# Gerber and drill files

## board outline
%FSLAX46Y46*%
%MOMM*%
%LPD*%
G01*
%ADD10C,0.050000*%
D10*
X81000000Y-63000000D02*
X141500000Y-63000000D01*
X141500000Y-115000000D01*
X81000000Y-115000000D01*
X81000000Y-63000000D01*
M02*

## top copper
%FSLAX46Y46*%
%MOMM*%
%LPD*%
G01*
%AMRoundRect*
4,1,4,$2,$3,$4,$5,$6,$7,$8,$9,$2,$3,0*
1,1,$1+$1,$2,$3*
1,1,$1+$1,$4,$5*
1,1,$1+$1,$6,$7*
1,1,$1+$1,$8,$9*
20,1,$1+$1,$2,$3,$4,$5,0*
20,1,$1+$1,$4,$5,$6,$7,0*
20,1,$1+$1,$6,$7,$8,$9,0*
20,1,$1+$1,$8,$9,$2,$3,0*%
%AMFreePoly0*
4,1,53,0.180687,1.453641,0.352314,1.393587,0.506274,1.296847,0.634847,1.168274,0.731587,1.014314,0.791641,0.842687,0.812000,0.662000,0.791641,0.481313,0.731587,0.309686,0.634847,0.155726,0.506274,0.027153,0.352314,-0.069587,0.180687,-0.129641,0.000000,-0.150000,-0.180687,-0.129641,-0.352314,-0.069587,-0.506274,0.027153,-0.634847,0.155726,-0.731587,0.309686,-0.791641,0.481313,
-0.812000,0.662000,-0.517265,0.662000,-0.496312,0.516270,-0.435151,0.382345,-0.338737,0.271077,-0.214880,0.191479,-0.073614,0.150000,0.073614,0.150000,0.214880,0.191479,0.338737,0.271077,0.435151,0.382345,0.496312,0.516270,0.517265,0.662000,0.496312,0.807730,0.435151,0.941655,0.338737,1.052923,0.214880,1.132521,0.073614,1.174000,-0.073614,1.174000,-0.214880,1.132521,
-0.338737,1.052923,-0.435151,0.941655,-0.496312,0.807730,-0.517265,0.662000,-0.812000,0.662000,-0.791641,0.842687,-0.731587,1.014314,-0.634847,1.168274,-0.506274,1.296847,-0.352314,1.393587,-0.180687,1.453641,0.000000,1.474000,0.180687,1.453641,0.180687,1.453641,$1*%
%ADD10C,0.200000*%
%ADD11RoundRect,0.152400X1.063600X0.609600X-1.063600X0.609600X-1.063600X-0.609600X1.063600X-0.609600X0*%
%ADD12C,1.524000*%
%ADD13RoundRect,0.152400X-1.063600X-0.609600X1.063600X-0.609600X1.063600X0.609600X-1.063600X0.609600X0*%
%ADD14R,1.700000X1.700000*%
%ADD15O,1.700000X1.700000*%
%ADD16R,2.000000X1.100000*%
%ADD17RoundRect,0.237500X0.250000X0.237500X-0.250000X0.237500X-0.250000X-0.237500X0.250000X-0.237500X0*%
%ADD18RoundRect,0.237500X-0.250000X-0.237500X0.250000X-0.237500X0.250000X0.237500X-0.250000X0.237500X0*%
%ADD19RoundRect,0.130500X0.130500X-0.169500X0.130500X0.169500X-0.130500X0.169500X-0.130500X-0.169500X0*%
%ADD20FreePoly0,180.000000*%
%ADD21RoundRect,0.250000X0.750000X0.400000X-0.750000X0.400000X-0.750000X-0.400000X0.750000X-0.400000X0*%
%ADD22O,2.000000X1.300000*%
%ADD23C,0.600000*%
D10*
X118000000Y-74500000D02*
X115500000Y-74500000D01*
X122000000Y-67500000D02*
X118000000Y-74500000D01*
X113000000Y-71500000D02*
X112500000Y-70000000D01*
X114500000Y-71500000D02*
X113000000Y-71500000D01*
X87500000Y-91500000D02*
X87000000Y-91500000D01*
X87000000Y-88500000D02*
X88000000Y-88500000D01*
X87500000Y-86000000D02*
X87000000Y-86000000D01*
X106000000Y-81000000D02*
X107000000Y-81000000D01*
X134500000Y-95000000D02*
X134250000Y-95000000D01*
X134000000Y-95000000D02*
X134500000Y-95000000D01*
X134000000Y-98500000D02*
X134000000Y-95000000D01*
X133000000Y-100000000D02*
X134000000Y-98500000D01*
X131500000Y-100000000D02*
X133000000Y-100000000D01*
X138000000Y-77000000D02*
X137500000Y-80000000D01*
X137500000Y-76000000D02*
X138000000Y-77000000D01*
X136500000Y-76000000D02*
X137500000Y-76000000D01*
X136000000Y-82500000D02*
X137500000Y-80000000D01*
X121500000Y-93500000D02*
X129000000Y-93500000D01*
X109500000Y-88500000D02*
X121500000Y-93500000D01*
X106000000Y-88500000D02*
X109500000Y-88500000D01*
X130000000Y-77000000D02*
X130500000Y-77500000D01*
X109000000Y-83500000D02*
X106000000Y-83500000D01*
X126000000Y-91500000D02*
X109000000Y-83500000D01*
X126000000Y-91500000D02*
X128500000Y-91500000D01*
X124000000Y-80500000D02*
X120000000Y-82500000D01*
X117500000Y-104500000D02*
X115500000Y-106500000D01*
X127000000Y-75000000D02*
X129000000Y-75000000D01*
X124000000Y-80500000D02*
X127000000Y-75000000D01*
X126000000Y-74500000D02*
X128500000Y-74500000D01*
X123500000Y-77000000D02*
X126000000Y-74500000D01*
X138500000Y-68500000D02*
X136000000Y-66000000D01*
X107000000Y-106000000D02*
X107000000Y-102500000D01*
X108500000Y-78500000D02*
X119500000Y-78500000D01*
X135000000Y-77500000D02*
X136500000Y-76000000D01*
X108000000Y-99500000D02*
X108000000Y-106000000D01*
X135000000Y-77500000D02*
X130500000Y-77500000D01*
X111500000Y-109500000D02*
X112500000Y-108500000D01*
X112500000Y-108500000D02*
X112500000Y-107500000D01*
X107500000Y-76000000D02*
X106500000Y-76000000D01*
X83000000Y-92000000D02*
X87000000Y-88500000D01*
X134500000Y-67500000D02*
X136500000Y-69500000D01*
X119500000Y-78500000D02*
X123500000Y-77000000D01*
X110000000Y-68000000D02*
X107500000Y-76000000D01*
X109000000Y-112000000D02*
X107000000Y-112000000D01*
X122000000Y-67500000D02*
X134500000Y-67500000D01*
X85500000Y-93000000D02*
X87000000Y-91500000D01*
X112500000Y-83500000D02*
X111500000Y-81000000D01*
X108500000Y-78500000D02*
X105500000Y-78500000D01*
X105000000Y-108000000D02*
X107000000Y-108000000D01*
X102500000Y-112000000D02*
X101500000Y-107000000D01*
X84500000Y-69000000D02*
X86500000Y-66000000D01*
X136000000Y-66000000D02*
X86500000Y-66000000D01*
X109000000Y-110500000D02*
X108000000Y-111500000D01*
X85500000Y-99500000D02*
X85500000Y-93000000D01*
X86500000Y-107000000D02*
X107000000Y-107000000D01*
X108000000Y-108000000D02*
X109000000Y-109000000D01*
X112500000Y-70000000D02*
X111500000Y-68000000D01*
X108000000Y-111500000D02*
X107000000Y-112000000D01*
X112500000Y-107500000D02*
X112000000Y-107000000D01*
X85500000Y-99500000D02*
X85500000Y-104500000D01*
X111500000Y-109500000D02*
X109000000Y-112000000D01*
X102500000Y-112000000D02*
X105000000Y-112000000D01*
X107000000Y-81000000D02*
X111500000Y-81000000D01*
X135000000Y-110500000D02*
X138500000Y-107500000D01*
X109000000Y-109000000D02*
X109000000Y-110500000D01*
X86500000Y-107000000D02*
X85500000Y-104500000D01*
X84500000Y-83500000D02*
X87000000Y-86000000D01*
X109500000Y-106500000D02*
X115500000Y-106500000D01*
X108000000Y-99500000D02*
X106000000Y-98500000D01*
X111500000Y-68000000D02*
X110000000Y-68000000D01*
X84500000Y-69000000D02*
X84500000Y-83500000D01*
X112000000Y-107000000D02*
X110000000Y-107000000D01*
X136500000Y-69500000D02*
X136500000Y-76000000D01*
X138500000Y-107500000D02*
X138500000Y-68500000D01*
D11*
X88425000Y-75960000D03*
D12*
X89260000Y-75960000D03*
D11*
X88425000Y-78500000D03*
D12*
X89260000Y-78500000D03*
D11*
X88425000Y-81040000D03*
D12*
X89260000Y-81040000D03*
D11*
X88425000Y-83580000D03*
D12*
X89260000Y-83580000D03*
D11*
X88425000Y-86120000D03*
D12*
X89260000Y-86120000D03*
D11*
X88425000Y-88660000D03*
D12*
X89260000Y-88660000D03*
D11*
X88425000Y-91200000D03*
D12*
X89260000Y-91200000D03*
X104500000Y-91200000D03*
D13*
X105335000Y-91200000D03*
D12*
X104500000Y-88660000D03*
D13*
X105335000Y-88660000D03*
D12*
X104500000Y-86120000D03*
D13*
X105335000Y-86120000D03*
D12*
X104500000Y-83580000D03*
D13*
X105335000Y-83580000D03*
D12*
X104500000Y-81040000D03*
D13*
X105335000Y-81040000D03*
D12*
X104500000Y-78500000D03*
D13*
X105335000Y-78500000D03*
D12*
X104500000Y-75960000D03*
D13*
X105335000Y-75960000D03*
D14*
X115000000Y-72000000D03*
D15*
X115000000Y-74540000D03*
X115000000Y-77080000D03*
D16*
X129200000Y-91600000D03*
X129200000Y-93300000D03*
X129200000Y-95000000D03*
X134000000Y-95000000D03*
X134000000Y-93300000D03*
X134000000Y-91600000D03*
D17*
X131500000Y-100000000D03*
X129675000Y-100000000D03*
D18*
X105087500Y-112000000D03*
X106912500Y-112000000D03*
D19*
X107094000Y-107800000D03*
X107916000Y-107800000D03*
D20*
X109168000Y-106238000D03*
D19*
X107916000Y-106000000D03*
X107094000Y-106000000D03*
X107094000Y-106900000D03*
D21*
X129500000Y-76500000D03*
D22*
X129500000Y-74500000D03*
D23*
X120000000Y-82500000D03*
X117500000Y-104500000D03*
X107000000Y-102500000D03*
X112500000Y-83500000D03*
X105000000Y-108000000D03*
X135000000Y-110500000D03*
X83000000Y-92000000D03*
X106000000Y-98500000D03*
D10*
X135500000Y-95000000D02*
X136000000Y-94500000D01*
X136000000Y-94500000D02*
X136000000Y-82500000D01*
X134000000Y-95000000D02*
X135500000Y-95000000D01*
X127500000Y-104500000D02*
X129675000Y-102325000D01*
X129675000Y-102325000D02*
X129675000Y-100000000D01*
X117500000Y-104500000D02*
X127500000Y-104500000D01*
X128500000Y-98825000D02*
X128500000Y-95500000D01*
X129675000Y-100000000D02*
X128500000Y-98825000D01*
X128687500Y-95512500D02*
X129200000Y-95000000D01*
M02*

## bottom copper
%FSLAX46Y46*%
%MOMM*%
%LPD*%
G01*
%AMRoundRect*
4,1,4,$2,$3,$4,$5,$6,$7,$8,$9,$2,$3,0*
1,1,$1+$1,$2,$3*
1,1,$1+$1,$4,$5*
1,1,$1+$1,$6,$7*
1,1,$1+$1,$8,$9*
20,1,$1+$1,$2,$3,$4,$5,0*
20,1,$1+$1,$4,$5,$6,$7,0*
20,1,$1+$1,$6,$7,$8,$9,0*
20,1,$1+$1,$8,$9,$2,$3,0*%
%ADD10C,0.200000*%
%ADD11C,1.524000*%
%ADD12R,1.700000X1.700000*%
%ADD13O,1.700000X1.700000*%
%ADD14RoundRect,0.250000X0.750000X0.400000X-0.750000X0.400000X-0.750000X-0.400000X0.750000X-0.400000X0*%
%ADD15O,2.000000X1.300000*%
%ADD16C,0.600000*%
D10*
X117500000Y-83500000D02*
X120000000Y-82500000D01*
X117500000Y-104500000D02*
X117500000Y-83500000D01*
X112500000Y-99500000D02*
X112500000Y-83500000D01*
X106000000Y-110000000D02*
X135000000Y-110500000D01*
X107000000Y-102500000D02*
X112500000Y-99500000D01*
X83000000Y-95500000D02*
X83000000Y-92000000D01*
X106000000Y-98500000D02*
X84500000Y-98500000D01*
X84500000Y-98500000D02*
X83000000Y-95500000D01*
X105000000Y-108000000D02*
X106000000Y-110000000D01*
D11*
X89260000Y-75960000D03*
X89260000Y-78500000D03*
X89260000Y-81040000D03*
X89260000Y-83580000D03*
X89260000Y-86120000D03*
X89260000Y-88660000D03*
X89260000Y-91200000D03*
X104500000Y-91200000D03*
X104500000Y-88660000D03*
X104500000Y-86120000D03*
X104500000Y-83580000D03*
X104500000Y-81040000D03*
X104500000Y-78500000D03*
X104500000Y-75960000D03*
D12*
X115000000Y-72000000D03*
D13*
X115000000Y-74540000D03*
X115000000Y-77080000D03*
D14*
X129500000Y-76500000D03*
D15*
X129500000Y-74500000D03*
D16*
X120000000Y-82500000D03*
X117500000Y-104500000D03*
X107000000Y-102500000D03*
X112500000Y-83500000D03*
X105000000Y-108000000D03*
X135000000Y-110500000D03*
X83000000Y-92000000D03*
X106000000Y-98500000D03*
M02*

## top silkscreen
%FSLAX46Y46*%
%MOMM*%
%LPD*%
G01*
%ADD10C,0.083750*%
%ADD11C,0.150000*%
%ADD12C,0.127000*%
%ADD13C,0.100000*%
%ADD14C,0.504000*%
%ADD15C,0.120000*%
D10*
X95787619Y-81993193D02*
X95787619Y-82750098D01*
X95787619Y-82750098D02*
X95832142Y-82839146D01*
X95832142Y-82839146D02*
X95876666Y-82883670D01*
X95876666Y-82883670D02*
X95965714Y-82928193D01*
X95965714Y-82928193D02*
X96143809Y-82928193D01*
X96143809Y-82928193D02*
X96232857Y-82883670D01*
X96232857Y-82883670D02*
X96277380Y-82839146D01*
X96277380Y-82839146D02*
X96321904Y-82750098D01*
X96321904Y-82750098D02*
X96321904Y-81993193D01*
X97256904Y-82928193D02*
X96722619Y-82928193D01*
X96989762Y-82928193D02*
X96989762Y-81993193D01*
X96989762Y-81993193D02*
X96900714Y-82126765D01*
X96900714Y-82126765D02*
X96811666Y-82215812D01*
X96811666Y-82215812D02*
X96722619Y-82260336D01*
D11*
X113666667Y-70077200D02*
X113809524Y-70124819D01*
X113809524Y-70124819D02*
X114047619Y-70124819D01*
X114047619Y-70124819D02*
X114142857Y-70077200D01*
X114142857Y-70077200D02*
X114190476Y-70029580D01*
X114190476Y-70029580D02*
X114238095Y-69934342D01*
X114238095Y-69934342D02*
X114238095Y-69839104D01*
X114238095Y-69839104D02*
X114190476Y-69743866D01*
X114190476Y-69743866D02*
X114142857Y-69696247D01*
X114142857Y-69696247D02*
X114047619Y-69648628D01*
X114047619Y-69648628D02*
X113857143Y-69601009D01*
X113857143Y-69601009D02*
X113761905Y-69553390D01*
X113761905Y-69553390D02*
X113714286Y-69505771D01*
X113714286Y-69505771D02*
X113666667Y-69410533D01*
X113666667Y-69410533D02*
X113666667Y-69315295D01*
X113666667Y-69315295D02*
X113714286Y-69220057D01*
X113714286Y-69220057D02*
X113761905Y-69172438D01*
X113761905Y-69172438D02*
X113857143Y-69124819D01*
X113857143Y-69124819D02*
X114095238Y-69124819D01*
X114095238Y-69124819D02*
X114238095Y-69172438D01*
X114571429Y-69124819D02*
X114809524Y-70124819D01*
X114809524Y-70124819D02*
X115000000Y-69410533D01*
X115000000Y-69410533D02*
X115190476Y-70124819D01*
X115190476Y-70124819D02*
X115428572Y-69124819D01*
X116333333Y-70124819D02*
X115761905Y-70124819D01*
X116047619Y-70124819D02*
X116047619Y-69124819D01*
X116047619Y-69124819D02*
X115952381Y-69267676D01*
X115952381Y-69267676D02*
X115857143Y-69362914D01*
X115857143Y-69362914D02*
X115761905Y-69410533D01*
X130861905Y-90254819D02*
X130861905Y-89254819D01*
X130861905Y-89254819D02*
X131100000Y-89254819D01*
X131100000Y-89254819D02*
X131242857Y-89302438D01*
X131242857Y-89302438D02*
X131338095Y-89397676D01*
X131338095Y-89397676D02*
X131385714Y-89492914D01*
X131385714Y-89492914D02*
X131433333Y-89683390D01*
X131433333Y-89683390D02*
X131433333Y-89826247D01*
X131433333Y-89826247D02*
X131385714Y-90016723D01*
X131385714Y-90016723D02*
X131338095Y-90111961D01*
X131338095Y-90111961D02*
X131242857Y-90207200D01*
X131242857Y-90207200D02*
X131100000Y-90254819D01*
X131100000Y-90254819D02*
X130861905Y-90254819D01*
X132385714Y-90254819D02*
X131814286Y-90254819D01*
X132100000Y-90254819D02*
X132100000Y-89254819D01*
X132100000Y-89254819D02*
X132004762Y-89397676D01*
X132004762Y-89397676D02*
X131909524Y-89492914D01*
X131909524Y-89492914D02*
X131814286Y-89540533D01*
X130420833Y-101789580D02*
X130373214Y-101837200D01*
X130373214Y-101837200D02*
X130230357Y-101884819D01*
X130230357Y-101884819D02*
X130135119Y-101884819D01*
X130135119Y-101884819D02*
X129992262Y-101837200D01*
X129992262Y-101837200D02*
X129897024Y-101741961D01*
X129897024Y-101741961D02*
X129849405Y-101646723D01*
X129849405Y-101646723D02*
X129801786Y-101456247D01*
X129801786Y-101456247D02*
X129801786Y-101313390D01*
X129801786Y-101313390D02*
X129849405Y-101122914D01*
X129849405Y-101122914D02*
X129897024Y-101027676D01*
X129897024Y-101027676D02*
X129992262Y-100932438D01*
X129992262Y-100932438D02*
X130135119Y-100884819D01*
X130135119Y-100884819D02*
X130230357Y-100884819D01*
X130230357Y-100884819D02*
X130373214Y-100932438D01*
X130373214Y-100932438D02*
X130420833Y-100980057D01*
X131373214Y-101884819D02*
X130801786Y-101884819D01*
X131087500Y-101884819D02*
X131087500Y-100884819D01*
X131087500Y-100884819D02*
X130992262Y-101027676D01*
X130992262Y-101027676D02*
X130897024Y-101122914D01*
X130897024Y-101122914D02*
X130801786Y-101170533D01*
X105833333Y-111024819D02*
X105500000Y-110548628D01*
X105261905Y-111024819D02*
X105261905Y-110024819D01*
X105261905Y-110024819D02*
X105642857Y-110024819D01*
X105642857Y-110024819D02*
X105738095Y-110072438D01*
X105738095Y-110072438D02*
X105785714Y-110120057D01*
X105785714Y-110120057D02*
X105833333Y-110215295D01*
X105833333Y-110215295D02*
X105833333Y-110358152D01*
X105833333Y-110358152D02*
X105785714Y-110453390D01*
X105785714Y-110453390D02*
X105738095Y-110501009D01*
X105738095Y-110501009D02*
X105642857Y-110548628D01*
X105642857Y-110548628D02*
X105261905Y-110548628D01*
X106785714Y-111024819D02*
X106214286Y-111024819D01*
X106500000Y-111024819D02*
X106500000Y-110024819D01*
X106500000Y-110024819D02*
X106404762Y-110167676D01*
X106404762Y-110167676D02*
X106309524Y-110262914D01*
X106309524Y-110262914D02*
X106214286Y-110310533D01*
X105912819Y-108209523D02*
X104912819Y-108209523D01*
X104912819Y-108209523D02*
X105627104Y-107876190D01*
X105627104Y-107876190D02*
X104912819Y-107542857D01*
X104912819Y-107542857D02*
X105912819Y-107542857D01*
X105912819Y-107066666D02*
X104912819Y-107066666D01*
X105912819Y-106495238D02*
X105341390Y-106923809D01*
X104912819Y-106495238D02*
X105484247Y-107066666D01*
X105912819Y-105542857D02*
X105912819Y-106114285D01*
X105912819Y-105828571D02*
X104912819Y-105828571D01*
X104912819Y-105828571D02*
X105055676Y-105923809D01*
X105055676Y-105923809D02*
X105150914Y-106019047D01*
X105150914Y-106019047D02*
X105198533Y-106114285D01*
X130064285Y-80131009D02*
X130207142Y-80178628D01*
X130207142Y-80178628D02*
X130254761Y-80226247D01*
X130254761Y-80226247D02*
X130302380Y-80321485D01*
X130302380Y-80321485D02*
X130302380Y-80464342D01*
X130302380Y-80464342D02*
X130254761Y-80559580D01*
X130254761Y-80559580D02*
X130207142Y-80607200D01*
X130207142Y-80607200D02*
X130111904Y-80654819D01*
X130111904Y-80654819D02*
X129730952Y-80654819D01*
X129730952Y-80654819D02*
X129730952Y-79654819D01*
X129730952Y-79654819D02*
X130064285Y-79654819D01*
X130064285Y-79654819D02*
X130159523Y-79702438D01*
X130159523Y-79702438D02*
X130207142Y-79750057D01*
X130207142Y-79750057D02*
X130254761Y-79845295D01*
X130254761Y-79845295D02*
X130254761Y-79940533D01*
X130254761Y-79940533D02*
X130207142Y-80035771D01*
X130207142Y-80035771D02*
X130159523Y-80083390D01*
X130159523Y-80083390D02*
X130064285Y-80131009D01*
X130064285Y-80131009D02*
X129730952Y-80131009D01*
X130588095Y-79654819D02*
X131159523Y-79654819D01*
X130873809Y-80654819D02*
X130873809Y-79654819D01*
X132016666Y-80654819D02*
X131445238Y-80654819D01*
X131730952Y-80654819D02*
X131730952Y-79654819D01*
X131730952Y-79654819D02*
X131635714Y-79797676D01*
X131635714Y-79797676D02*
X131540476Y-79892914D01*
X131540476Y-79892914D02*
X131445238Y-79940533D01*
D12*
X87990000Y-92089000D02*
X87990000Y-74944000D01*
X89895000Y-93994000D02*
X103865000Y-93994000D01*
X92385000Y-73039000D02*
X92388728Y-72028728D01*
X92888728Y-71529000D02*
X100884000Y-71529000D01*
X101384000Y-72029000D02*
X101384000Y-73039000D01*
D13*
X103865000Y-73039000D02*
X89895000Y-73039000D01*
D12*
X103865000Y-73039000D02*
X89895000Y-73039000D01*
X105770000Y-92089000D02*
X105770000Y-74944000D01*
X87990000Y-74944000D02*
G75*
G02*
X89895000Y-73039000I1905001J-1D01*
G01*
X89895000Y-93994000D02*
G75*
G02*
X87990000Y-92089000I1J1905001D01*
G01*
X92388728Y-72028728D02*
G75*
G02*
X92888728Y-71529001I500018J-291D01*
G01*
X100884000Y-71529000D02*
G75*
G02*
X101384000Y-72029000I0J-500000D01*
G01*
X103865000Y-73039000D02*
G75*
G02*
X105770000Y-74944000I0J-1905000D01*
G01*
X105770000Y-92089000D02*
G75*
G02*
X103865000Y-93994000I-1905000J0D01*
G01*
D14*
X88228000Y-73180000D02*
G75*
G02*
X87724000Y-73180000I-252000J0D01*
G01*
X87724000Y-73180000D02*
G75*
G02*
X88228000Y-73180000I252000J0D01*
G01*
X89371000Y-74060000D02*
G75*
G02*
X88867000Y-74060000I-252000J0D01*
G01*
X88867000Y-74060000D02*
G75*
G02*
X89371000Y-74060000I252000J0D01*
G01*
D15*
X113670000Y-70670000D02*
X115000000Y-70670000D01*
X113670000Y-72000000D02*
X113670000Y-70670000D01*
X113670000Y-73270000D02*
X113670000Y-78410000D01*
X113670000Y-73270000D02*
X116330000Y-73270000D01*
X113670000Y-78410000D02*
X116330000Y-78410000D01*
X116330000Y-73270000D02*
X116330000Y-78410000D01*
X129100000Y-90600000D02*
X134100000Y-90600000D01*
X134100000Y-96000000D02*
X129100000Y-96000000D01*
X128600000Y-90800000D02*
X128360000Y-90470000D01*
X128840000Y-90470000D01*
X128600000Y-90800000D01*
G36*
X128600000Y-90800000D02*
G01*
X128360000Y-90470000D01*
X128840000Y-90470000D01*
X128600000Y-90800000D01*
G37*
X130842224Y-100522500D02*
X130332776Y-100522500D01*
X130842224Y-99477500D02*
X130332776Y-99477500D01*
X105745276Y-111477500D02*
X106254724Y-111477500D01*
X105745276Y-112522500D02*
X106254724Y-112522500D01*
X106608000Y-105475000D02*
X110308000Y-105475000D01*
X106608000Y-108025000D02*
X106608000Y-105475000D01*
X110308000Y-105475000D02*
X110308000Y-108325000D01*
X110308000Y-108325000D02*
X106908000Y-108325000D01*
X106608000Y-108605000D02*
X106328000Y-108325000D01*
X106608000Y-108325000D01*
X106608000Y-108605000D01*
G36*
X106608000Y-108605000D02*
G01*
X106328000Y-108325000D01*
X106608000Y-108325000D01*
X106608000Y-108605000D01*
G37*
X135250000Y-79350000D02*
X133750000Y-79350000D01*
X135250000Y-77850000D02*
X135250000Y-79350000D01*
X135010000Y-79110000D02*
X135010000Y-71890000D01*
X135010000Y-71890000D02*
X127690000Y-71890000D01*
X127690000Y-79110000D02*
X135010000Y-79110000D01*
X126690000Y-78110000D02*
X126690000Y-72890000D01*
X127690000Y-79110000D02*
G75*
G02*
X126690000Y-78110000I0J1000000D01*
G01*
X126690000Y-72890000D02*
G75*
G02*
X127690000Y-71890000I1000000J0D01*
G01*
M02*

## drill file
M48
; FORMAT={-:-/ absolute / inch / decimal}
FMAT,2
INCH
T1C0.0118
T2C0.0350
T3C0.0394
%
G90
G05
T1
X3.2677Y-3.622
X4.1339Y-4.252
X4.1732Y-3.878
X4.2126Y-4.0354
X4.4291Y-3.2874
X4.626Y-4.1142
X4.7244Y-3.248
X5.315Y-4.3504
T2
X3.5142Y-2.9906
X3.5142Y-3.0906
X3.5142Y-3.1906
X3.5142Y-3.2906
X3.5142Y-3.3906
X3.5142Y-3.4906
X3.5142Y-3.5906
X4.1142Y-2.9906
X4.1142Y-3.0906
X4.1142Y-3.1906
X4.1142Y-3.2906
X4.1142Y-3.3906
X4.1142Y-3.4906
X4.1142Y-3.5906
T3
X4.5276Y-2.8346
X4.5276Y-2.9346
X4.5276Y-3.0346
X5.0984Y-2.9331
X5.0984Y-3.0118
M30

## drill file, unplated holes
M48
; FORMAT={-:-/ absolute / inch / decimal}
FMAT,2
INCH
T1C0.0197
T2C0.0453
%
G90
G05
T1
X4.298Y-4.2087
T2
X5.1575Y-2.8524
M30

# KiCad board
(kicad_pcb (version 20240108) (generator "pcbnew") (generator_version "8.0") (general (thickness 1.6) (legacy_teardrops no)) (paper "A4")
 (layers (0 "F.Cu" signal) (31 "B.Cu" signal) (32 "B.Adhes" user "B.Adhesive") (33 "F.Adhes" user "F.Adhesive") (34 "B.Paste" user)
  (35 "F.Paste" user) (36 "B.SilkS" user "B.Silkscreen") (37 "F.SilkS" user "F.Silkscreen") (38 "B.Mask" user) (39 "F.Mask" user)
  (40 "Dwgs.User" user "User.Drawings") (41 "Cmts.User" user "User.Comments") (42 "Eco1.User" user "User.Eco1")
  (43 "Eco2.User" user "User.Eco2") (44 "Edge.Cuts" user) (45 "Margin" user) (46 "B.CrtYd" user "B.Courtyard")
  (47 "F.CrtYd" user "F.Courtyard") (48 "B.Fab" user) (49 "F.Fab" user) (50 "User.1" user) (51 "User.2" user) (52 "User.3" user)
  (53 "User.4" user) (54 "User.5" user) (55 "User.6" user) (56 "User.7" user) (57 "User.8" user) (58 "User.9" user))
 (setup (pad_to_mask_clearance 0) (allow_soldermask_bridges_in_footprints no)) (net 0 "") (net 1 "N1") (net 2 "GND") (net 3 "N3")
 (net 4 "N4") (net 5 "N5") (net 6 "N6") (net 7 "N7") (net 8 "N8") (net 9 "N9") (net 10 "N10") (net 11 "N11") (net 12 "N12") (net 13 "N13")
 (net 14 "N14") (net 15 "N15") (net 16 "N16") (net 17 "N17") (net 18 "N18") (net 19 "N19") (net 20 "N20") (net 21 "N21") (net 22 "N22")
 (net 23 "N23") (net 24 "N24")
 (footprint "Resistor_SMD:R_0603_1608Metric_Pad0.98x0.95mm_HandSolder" (layer "F.Cu") (at 130.5875 100 180)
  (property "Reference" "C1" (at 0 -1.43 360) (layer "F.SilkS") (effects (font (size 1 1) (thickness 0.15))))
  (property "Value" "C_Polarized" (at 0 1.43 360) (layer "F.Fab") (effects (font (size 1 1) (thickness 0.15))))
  (fp_line (start -0.254724 0.5225) (end 0.254724 0.5225) (stroke (width 0.12) (type solid)) (layer "F.SilkS"))
  (fp_line (start -0.254724 -0.5225) (end 0.254724 -0.5225) (stroke (width 0.12) (type solid)) (layer "F.SilkS"))
  (pad "1" smd roundrect (at -0.9125 0 180) (size 0.975 0.95) (layers "F.Cu" "F.Paste" "F.Mask") (roundrect_rratio 0.25) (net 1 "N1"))
  (pad "2" smd roundrect (at 0.9125 0 180) (size 0.975 0.95) (layers "F.Cu" "F.Paste" "F.Mask") (roundrect_rratio 0.25) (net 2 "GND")))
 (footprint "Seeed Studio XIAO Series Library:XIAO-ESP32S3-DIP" (layer "F.Cu") (at 96.88 83.58)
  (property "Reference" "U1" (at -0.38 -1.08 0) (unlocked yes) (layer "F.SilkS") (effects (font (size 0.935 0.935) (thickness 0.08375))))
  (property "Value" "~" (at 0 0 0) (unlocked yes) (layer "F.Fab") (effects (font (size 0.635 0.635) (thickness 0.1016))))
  (fp_line (start -8.89 8.509) (end -8.89 -8.636) (stroke (width 0.127) (type solid)) (layer "F.SilkS"))
  (fp_line (start -6.985 10.414) (end 6.985 10.414) (stroke (width 0.127) (type solid)) (layer "F.SilkS"))
  (fp_line (start -4.495 -10.541) (end -4.491272 -11.551272) (stroke (width 0.127) (type solid)) (layer "F.SilkS"))
  (fp_line (start -3.991272 -12.051) (end 4.004 -12.051) (stroke (width 0.127) (type solid)) (layer "F.SilkS"))
  (fp_line (start 4.504 -11.551) (end 4.504 -10.541) (stroke (width 0.127) (type solid)) (layer "F.SilkS"))
  (fp_line (start 6.985 -10.541) (end -6.985 -10.541) (stroke (width 0.1) (type solid)) (layer "F.SilkS"))
  (fp_line (start 6.985 -10.541) (end -6.985 -10.541) (stroke (width 0.127) (type solid)) (layer "F.SilkS"))
  (fp_line (start 8.89 8.509) (end 8.89 -8.636) (stroke (width 0.127) (type solid)) (layer "F.SilkS"))
  (fp_arc (start -8.89 -8.636) (mid -8.332038 -9.983038) (end -6.985 -10.541) (stroke (width 0.127) (type solid)) (layer "F.SilkS"))
  (fp_arc (start -6.985 10.414) (mid -8.332038 9.856038) (end -8.89 8.509) (stroke (width 0.127) (type solid)) (layer "F.SilkS"))
  (fp_arc (start -4.491272 -11.551272) (mid -4.344724 -11.904644) (end -3.991272 -12.051) (stroke (width 0.127) (type default))
   (layer "F.SilkS"))
  (fp_arc (start 4.004 -12.051) (mid 4.357553 -11.904553) (end 4.504 -11.551) (stroke (width 0.127) (type default)) (layer "F.SilkS"))
  (fp_arc (start 6.985 -10.541) (mid 8.332038 -9.983038) (end 8.89 -8.636) (stroke (width 0.127) (type solid)) (layer "F.SilkS"))
  (fp_arc (start 8.89 8.509) (mid 8.332038 9.856038) (end 6.985 10.414) (stroke (width 0.127) (type solid)) (layer "F.SilkS"))
  (fp_circle (center -8.904 -10.4) (end -8.904 -10.654) (stroke (width 0.5) (type solid)) (fill solid) (layer "F.SilkS"))
  (fp_circle (center -7.761 -9.52) (end -7.761 -9.774) (stroke (width 0.5) (type solid)) (fill solid) (layer "F.SilkS"))
  (pad "1" smd roundrect (at -8.455 -7.62 180) (size 2.432 1.524) (layers "F.Cu" "F.Mask") (roundrect_rratio 0.1) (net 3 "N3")
   (thermal_bridge_angle 45))
  (pad "1" thru_hole circle (at -7.62 -7.62 180) (size 1.524 1.524) (drill 0.889) (layers "*.Cu" "*.Mask") (remove_unused_layers no)
   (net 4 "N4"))
  (pad "2" smd roundrect (at -8.455 -5.08 180) (size 2.432 1.524) (layers "F.Cu" "F.Mask") (roundrect_rratio 0.1) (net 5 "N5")
   (thermal_bridge_angle 45))
  (pad "2" thru_hole circle (at -7.62 -5.08 180) (size 1.524 1.524) (drill 0.889) (layers "*.Cu" "*.Mask") (remove_unused_layers no)
   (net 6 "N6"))
  (pad "3" smd roundrect (at -8.455 -2.54 180) (size 2.432 1.524) (layers "F.Cu" "F.Mask") (roundrect_rratio 0.1) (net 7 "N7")
   (thermal_bridge_angle 45))
  (pad "3" thru_hole circle (at -7.62 -2.54 180) (size 1.524 1.524) (drill 0.889) (layers "*.Cu" "*.Mask") (remove_unused_layers no)
   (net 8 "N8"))
  (pad "4" smd roundrect (at -8.455 0 180) (size 2.432 1.524) (layers "F.Cu" "F.Mask") (roundrect_rratio 0.1) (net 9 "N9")
   (thermal_bridge_angle 45))
  (pad "4" thru_hole circle (at -7.62 0 180) (size 1.524 1.524) (drill 0.889) (layers "*.Cu" "*.Mask") (remove_unused_layers no)
   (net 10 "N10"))
  (pad "5" smd roundrect (at -8.455 2.54 180) (size 2.432 1.524) (layers "F.Cu" "F.Mask") (roundrect_rratio 0.1) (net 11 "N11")
   (thermal_bridge_angle 45))
  (pad "5" thru_hole circle (at -7.62 2.54 180) (size 1.524 1.524) (drill 0.889) (layers "*.Cu" "*.Mask") (remove_unused_layers no)
   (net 11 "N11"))
  (pad "6" smd roundrect (at -8.455 5.08 180) (size 2.432 1.524) (layers "F.Cu" "F.Mask") (roundrect_rratio 0.1) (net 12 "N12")
   (thermal_bridge_angle 45))
  (pad "6" thru_hole circle (at -7.62 5.08 180) (size 1.524 1.524) (drill 0.889) (layers "*.Cu" "*.Mask") (remove_unused_layers no)
   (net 12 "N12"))
  (pad "7" smd roundrect (at -8.455 7.62 180) (size 2.432 1.524) (layers "F.Cu" "F.Mask") (roundrect_rratio 0.1) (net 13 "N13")
   (thermal_bridge_angle 45))
  (pad "7" thru_hole circle (at -7.62 7.62 180) (size 1.524 1.524) (drill 0.889) (layers "*.Cu" "*.Mask") (remove_unused_layers no)
   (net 13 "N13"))
  (pad "8" thru_hole circle (at 7.62 7.62) (size 1.524 1.524) (drill 0.889) (layers "*.Cu" "*.Mask") (remove_unused_layers no)
   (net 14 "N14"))
  (pad "8" smd roundrect (at 8.455 7.62) (size 2.432 1.524) (layers "F.Cu" "F.Mask") (roundrect_rratio 0.1) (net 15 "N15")
   (thermal_bridge_angle 45))
  (pad "9" thru_hole circle (at 7.62 5.08) (size 1.524 1.524) (drill 0.889) (layers "*.Cu" "*.Mask") (remove_unused_layers no)
   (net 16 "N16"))
  (pad "9" smd roundrect (at 8.455 5.08) (size 2.432 1.524) (layers "F.Cu" "F.Mask") (roundrect_rratio 0.1) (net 16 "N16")
   (thermal_bridge_angle 45))
  (pad "10" thru_hole circle (at 7.62 2.54) (size 1.524 1.524) (drill 0.889) (layers "*.Cu" "*.Mask") (remove_unused_layers no)
   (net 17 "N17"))
  (pad "10" smd roundrect (at 8.455 2.54) (size 2.432 1.524) (layers "F.Cu" "F.Mask") (roundrect_rratio 0.1) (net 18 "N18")
   (thermal_bridge_angle 45))
  (pad "11" thru_hole circle (at 7.62 0) (size 1.524 1.524) (drill 0.889) (layers "*.Cu" "*.Mask") (remove_unused_layers no) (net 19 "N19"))
  (pad "11" smd roundrect (at 8.455 0) (size 2.432 1.524) (layers "F.Cu" "F.Mask") (roundrect_rratio 0.1) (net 19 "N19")
   (thermal_bridge_angle 45))
  (pad "12" thru_hole circle (at 7.62 -2.54) (size 1.524 1.524) (drill 0.889) (layers "*.Cu" "*.Mask") (remove_unused_layers no)
   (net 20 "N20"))
  (pad "12" smd roundrect (at 8.455 -2.54) (size 2.432 1.524) (layers "F.Cu" "F.Mask") (roundrect_rratio 0.1) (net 20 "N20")
   (thermal_bridge_angle 45))
  (pad "13" thru_hole circle (at 7.62 -5.08) (size 1.524 1.524) (drill 0.889) (layers "*.Cu" "*.Mask") (remove_unused_layers no)
   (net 2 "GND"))
  (pad "13" smd roundrect (at 8.455 -5.08) (size 2.432 1.524) (layers "F.Cu" "F.Mask") (roundrect_rratio 0.1) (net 2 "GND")
   (thermal_bridge_angle 45))
  (pad "14" thru_hole circle (at 7.62 -7.62) (size 1.524 1.524) (drill 0.889) (layers "*.Cu" "*.Mask") (remove_unused_layers no)
   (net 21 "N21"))
  (pad "14" smd roundrect (at 8.455 -7.62) (size 2.432 1.524) (layers "F.Cu" "F.Mask") (roundrect_rratio 0.1) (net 21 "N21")
   (thermal_bridge_angle 45)))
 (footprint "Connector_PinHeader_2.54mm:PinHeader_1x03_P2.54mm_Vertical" (layer "F.Cu") (at 115 72)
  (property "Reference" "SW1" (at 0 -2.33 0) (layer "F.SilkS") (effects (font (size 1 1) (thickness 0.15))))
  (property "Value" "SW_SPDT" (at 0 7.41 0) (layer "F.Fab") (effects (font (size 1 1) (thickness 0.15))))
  (fp_line (start -1.33 -1.33) (end 0 -1.33) (stroke (width 0.12) (type solid)) (layer "F.SilkS"))
  (fp_line (start -1.33 0) (end -1.33 -1.33) (stroke (width 0.12) (type solid)) (layer "F.SilkS"))
  (fp_line (start -1.33 1.27) (end -1.33 6.41) (stroke (width 0.12) (type solid)) (layer "F.SilkS"))
  (fp_line (start -1.33 1.27) (end 1.33 1.27) (stroke (width 0.12) (type solid)) (layer "F.SilkS"))
  (fp_line (start -1.33 6.41) (end 1.33 6.41) (stroke (width 0.12) (type solid)) (layer "F.SilkS"))
  (fp_line (start 1.33 1.27) (end 1.33 6.41) (stroke (width 0.12) (type solid)) (layer "F.SilkS"))
  (pad "1" thru_hole rect (at 0 0) (size 1.7 1.7) (drill 1) (layers "*.Cu" "*.Mask") (remove_unused_layers no) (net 21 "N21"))
  (pad "2" thru_hole oval (at 0 2.54) (size 1.7 1.7) (drill 1) (layers "*.Cu" "*.Mask") (remove_unused_layers no) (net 1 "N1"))
  (pad "3" thru_hole oval (at 0 5.08) (size 1.7 1.7) (drill 1) (layers "*.Cu" "*.Mask") (remove_unused_layers no) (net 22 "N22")))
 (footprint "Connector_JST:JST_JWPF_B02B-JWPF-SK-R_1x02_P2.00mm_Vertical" (layer "F.Cu") (at 129.5 76.5 180)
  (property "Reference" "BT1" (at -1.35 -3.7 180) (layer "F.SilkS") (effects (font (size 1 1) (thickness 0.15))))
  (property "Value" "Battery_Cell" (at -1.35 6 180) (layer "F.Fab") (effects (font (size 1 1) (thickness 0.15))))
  (fp_line (start 2.81 -1.61) (end 2.81 3.61) (stroke (width 0.12) (type solid)) (layer "F.SilkS"))
  (fp_line (start 1.81 -2.61) (end -5.51 -2.61) (stroke (width 0.12) (type solid)) (layer "F.SilkS"))
  (fp_line (start -5.51 4.61) (end 1.81 4.61) (stroke (width 0.12) (type solid)) (layer "F.SilkS"))
  (fp_line (start -5.51 -2.61) (end -5.51 4.61) (stroke (width 0.12) (type solid)) (layer "F.SilkS"))
  (fp_line (start -5.75 -1.35) (end -5.75 -2.85) (stroke (width 0.12) (type solid)) (layer "F.SilkS"))
  (fp_line (start -5.75 -2.85) (end -4.25 -2.85) (stroke (width 0.12) (type solid)) (layer "F.SilkS"))
  (fp_arc (start 2.81 3.61) (mid 2.517107 4.317107) (end 1.81 4.61) (stroke (width 0.12) (type solid)) (layer "F.SilkS"))
  (fp_arc (start 1.81 -2.61) (mid 2.517107 -2.317107) (end 2.81 -1.61) (stroke (width 0.12) (type solid)) (layer "F.SilkS"))
  (pad "" np_thru_hole circle (at -1.5 4.05 180) (size 1.15 1.15) (drill 1.15) (layers "*.Cu" "*.Mask"))
  (pad "1" thru_hole roundrect (at 0 0 180) (size 2 1.3) (drill 1) (layers "*.Cu" "*.Mask") (remove_unused_layers no)
   (roundrect_rratio 0.192308) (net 1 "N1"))
  (pad "2" thru_hole oval (at 0 2 180) (size 2 1.3) (drill 1) (layers "*.Cu" "*.Mask") (remove_unused_layers no) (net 2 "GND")))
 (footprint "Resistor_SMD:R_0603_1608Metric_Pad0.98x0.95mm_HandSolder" (layer "F.Cu") (at 106 112)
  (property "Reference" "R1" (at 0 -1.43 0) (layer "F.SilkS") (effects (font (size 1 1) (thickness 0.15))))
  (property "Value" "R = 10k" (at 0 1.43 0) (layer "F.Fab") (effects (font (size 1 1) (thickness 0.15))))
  (fp_line (start -0.254724 -0.5225) (end 0.254724 -0.5225) (stroke (width 0.12) (type solid)) (layer "F.SilkS"))
  (fp_line (start -0.254724 0.5225) (end 0.254724 0.5225) (stroke (width 0.12) (type solid)) (layer "F.SilkS"))
  (pad "1" smd roundrect (at -0.9125 0) (size 0.975 0.95) (layers "F.Cu" "F.Paste" "F.Mask") (roundrect_rratio 0.25) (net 13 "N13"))
  (pad "2" smd roundrect (at 0.9125 0) (size 0.975 0.95) (layers "F.Cu" "F.Paste" "F.Mask") (roundrect_rratio 0.25) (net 2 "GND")))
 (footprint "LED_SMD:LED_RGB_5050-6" (layer "F.Cu") (at 131.6 93.3)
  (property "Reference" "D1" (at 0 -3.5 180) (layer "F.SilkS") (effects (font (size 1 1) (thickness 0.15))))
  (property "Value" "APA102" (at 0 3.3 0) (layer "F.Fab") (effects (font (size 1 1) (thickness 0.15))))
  (fp_line (start -2.5 -2.7) (end 2.5 -2.7) (stroke (width 0.12) (type solid)) (layer "F.SilkS"))
  (fp_line (start 2.5 2.7) (end -2.5 2.7) (stroke (width 0.12) (type solid)) (layer "F.SilkS"))
  (fp_poly
   (pts (xy -3 -2.5) (xy -3.24 -2.83) (xy -2.76 -2.83) (xy -3 -2.5)) (stroke (width 0.12) (type solid)) (fill solid) (layer "F.SilkS"))
  (pad "1" smd rect (at -2.4 -1.7 90) (size 1.1 2) (layers "F.Cu" "F.Paste" "F.Mask") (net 19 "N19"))
  (pad "2" smd rect (at -2.4 0 90) (size 1.1 2) (layers "F.Cu" "F.Paste" "F.Mask") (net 16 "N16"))
  (pad "3" smd rect (at -2.4 1.7 90) (size 1.1 2) (layers "F.Cu" "F.Paste" "F.Mask") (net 2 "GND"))
  (pad "4" smd rect (at 2.4 1.7 90) (size 1.1 2) (layers "F.Cu" "F.Paste" "F.Mask") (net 1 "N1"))
  (pad "5" smd rect (at 2.4 0 90) (size 1.1 2) (layers "F.Cu" "F.Paste" "F.Mask") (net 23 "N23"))
  (pad "6" smd rect (at 2.4 -1.7 90) (size 1.1 2) (layers "F.Cu" "F.Paste" "F.Mask") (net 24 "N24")))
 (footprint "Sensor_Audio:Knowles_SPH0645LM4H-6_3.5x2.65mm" (layer "F.Cu") (at 108.458 106.9 90)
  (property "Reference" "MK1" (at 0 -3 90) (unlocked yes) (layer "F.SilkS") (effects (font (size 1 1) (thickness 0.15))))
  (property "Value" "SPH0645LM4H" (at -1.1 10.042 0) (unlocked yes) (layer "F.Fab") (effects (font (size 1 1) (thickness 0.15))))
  (fp_line (start 1.425 -1.85) (end 1.425 1.85) (stroke (width 0.12) (type default)) (layer "F.SilkS"))
  (fp_line (start -1.125 -1.85) (end 1.425 -1.85) (stroke (width 0.12) (type default)) (layer "F.SilkS"))
  (fp_line (start 1.425 1.85) (end -1.425 1.85) (stroke (width 0.12) (type default)) (layer "F.SilkS"))
  (fp_line (start -1.425 1.85) (end -1.425 -1.55) (stroke (width 0.12) (type default)) (layer "F.SilkS"))
  (fp_poly
   (pts (xy -1.425 -1.85) (xy -1.705 -1.85) (xy -1.425 -2.13) (xy -1.425 -1.85)) (stroke (width 0.12) (type solid)) (fill solid)
   (layer "F.SilkS"))
  (pad "" np_thru_hole circle (at 0 0.71 90) (size 0.5 0.5) (drill 0.5) (layers "*.Mask"))
  (pad "1" smd roundrect (at -0.9 -1.364 90) (size 0.6 0.522) (layers "F.Cu" "F.Paste" "F.Mask") (roundrect_rratio 0.25) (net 11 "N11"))
  (pad "2" smd roundrect (at -0.9 -0.542 90) (size 0.6 0.522) (layers "F.Cu" "F.Paste" "F.Mask") (roundrect_rratio 0.25) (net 2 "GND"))
  (pad "3" smd custom (at 0.662 0.71 180) (size 0.3 0.3) (layers "F.Cu" "F.Mask") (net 2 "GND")
   (options (clearance outline) (anchor circle)) (primitives))
  (pad "4" smd roundrect (at 0.9 -0.542 90) (size 0.6 0.522) (layers "F.Cu" "F.Paste" "F.Mask") (roundrect_rratio 0.25) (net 12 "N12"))
  (pad "5" smd roundrect (at 0.9 -1.364 90) (size 0.6 0.522) (layers "F.Cu" "F.Paste" "F.Mask") (roundrect_rratio 0.25) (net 20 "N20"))
  (pad "6" smd roundrect (at 0 -1.364 90) (size 0.6 0.522) (layers "F.Cu" "F.Paste" "F.Mask") (roundrect_rratio 0.25) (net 13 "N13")))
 (gr_line (start 137.5 76) (end 138 77) (stroke (width 0.2) (type default)) (layer "F.Cu") (net 1))
 (gr_line (start 106 88.5) (end 109.5 88.5) (stroke (width 0.2) (type default)) (layer "F.Cu") (net 16))
 (gr_line (start 138.5 68.5) (end 136 66) (stroke (width 0.2) (type default)) (layer "F.Cu") (net 11))
 (gr_line (start 126 91.5) (end 109 83.5) (stroke (width 0.2) (type default)) (layer "F.Cu") (net 19))
 (gr_line (start 124 80.5) (end 127 75) (stroke (width 0.2) (type default)) (layer "F.Cu") (net 2))
 (gr_line (start 107 106) (end 107 102.5) (stroke (width 0.2) (type default)) (layer "F.Cu") (net 20))
 (gr_line (start 134 95) (end 134.5 95) (stroke (width 0.2) (type default)) (layer "F.Cu") (net 1))
 (gr_line (start 108.5 78.5) (end 119.5 78.5) (stroke (width 0.2) (type default)) (layer "F.Cu") (net 2))
 (gr_line (start 135 77.5) (end 136.5 76) (stroke (width 0.2) (type default)) (layer "F.Cu") (net 1))
 (gr_line (start 108 99.5) (end 108 106) (stroke (width 0.2) (type default)) (layer "F.Cu") (net 12))
 (gr_line (start 135 77.5) (end 130.5 77.5) (stroke (width 0.2) (type default)) (layer "F.Cu") (net 1))
 (gr_line (start 109.5 88.5) (end 121.5 93.5) (stroke (width 0.2) (type default)) (layer "F.Cu") (net 16))
 (gr_line (start 111.5 109.5) (end 112.5 108.5) (stroke (width 0.2) (type default)) (layer "F.Cu") (net 2))
 (gr_line (start 112.5 108.5) (end 112.5 107.5) (stroke (width 0.2) (type default)) (layer "F.Cu") (net 2))
 (gr_line (start 127 75) (end 129 75) (stroke (width 0.2) (type default)) (layer "F.Cu") (net 2))
 (gr_line (start 123.5 77) (end 126 74.5) (stroke (width 0.2) (type default)) (layer "F.Cu") (net 2))
 (gr_line (start 107.5 76) (end 106.5 76) (stroke (width 0.2) (type default)) (layer "F.Cu") (net 21))
 (gr_line (start 83 92) (end 87 88.5) (stroke (width 0.2) (type default)) (layer "F.Cu") (net 12))
 (gr_line (start 134.5 67.5) (end 136.5 69.5) (stroke (width 0.2) (type default)) (layer "F.Cu") (net 1))
 (gr_line (start 119.5 78.5) (end 123.5 77) (stroke (width 0.2) (type default)) (layer "F.Cu") (net 2))
 (gr_line (start 110 68) (end 107.5 76) (stroke (width 0.2) (type default)) (layer "F.Cu") (net 21))
 (gr_line (start 121.5 93.5) (end 129 93.5) (stroke (width 0.2) (type default)) (layer "F.Cu") (net 16))
 (gr_line (start 109 83.5) (end 106 83.5) (stroke (width 0.2) (type default)) (layer "F.Cu") (net 19))
 (gr_line (start 109 112) (end 107 112) (stroke (width 0.2) (type default)) (layer "F.Cu") (net 2))
 (gr_line (start 106 81) (end 107 81) (stroke (width 0.2) (type default)) (layer "F.Cu") (net 20))
 (gr_line (start 117.5 104.5) (end 115.5 106.5) (stroke (width 0.2) (type default)) (layer "F.Cu") (net 2))
 (gr_line (start 122 67.5) (end 134.5 67.5) (stroke (width 0.2) (type default)) (layer "F.Cu") (net 1))
 (gr_line (start 85.5 93) (end 87 91.5) (stroke (width 0.2) (type default)) (layer "F.Cu") (net 13))
 (gr_line (start 136 82.5) (end 137.5 80) (stroke (width 0.2) (type default)) (layer "F.Cu") (net 1))
 (gr_line (start 112.5 83.5) (end 111.5 81) (stroke (width 0.2) (type default)) (layer "F.Cu") (net 20))
 (gr_line (start 108.5 78.5) (end 105.5 78.5) (stroke (width 0.2) (type default)) (layer "F.Cu") (net 2))
 (gr_line (start 105 108) (end 107 108) (stroke (width 0.2) (type default)) (layer "F.Cu") (net 11))
 (gr_line (start 138 77) (end 137.5 80) (stroke (width 0.2) (type default)) (layer "F.Cu") (net 1))
 (gr_line (start 102.5 112) (end 101.5 107) (stroke (width 0.2) (type default)) (layer "F.Cu") (net 13))
 (gr_line (start 134.5 95) (end 134.25 95) (stroke (width 0.2) (type default)) (layer "F.Cu") (net 1))
 (gr_line (start 84.5 69) (end 86.5 66) (stroke (width 0.2) (type default)) (layer "F.Cu") (net 11))
 (gr_line (start 136 66) (end 86.5 66) (stroke (width 0.2) (type default)) (layer "F.Cu") (net 11))
 (gr_line (start 87.5 86) (end 87 86) (stroke (width 0.2) (type default)) (layer "F.Cu") (net 11))
 (gr_line (start 131.5 100) (end 133 100) (stroke (width 0.2) (type default)) (layer "F.Cu") (net 1))
 (gr_line (start 126 91.5) (end 128.5 91.5) (stroke (width 0.2) (type default)) (layer "F.Cu") (net 19))
 (gr_line (start 109 110.5) (end 108 111.5) (stroke (width 0.2) (type default)) (layer "F.Cu") (net 2))
 (gr_line (start 85.5 99.5) (end 85.5 93) (stroke (width 0.2) (type default)) (layer "F.Cu") (net 13))
 (gr_line (start 86.5 107) (end 107 107) (stroke (width 0.2) (type default)) (layer "F.Cu") (net 13))
 (gr_line (start 134 98.5) (end 134 95) (stroke (width 0.2) (type default)) (layer "F.Cu") (net 1))
 (gr_line (start 108 108) (end 109 109) (stroke (width 0.2) (type default)) (layer "F.Cu") (net 2))
 (gr_line (start 112.5 70) (end 111.5 68) (stroke (width 0.2) (type default)) (layer "F.Cu") (net 21))
 (gr_line (start 136.5 76) (end 137.5 76) (stroke (width 0.2) (type default)) (layer "F.Cu") (net 1))
 (gr_line (start 87 88.5) (end 88 88.5) (stroke (width 0.2) (type default)) (layer "F.Cu") (net 12))
 (gr_line (start 108 111.5) (end 107 112) (stroke (width 0.2) (type default)) (layer "F.Cu") (net 2))
 (gr_line (start 112.5 107.5) (end 112 107) (stroke (width 0.2) (type default)) (layer "F.Cu") (net 2))
 (gr_line (start 85.5 99.5) (end 85.5 104.5) (stroke (width 0.2) (type default)) (layer "F.Cu") (net 13))
 (gr_line (start 111.5 109.5) (end 109 112) (stroke (width 0.2) (type default)) (layer "F.Cu") (net 2))
 (gr_line (start 133 100) (end 134 98.5) (stroke (width 0.2) (type default)) (layer "F.Cu") (net 1))
 (gr_line (start 114.5 71.5) (end 113 71.5) (stroke (width 0.2) (type default)) (layer "F.Cu") (net 21))
 (gr_line (start 102.5 112) (end 105 112) (stroke (width 0.2) (type default)) (layer "F.Cu") (net 13))
 (gr_line (start 107 81) (end 111.5 81) (stroke (width 0.2) (type default)) (layer "F.Cu") (net 20))
 (gr_line (start 126 74.5) (end 128.5 74.5) (stroke (width 0.2) (type default)) (layer "F.Cu") (net 2))
 (gr_line (start 135 110.5) (end 138.5 107.5) (stroke (width 0.2) (type default)) (layer "F.Cu") (net 11))
 (gr_line (start 109 109) (end 109 110.5) (stroke (width 0.2) (type default)) (layer "F.Cu") (net 2))
 (gr_line (start 86.5 107) (end 85.5 104.5) (stroke (width 0.2) (type default)) (layer "F.Cu") (net 13))
 (gr_line (start 118 74.5) (end 115.5 74.5) (stroke (width 0.2) (type default)) (layer "F.Cu") (net 1))
 (gr_line (start 87.5 91.5) (end 87 91.5) (stroke (width 0.2) (type default)) (layer "F.Cu") (net 13))
 (gr_line (start 122 67.5) (end 118 74.5) (stroke (width 0.2) (type default)) (layer "F.Cu") (net 1))
 (gr_line (start 84.5 83.5) (end 87 86) (stroke (width 0.2) (type default)) (layer "F.Cu") (net 11))
 (gr_line (start 109.5 106.5) (end 115.5 106.5) (stroke (width 0.2) (type default)) (layer "F.Cu") (net 2))
 (gr_line (start 108 99.5) (end 106 98.5) (stroke (width 0.2) (type default)) (layer "F.Cu") (net 12))
 (gr_line (start 113 71.5) (end 112.5 70) (stroke (width 0.2) (type default)) (layer "F.Cu") (net 21))
 (gr_line (start 111.5 68) (end 110 68) (stroke (width 0.2) (type default)) (layer "F.Cu") (net 21))
 (gr_line (start 130 77) (end 130.5 77.5) (stroke (width 0.2) (type default)) (layer "F.Cu") (net 1))
 (gr_line (start 84.5 69) (end 84.5 83.5) (stroke (width 0.2) (type default)) (layer "F.Cu") (net 11))
 (gr_line (start 124 80.5) (end 120 82.5) (stroke (width 0.2) (type default)) (layer "F.Cu") (net 2))
 (gr_line (start 112 107) (end 110 107) (stroke (width 0.2) (type default)) (layer "F.Cu") (net 2))
 (gr_line (start 136.5 69.5) (end 136.5 76) (stroke (width 0.2) (type default)) (layer "F.Cu") (net 1))
 (gr_line (start 138.5 107.5) (end 138.5 68.5) (stroke (width 0.2) (type default)) (layer "F.Cu") (net 11))
 (gr_line (start 117.5 83.5) (end 120 82.5) (stroke (width 0.2) (type default)) (layer "B.Cu") (net 2))
 (gr_line (start 112.5 99.5) (end 112.5 83.5) (stroke (width 0.2) (type default)) (layer "B.Cu") (net 20))
 (gr_line (start 106 110) (end 135 110.5) (stroke (width 0.2) (type default)) (layer "B.Cu") (net 11))
 (gr_line (start 107 102.5) (end 112.5 99.5) (stroke (width 0.2) (type default)) (layer "B.Cu") (net 20))
 (gr_line (start 83 95.5) (end 83 92) (stroke (width 0.2) (type default)) (layer "B.Cu") (net 12))
 (gr_line (start 106 98.5) (end 84.5 98.5) (stroke (width 0.2) (type default)) (layer "B.Cu") (net 12))
 (gr_line (start 84.5 98.5) (end 83 95.5) (stroke (width 0.2) (type default)) (layer "B.Cu") (net 12))
 (gr_line (start 105 108) (end 106 110) (stroke (width 0.2) (type default)) (layer "B.Cu") (net 11))
 (gr_line (start 117.5 104.5) (end 117.5 83.5) (stroke (width 0.2) (type default)) (layer "B.Cu") (net 2))
 (gr_rect (start 81 63) (end 141.5 115) (stroke (width 0.05) (type default)) (fill none) (layer "Edge.Cuts"))
 (via (at 107 102.5) (size 0.6) (drill 0.3) (layers "F.Cu" "B.Cu") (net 20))
 (via (at 112.5 83.5) (size 0.6) (drill 0.3) (layers "F.Cu" "B.Cu") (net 20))
 (via (at 105 108) (size 0.6) (drill 0.3) (layers "F.Cu" "B.Cu") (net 11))
 (via (at 135 110.5) (size 0.6) (drill 0.3) (layers "F.Cu" "B.Cu") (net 11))
 (via (at 83 92) (size 0.6) (drill 0.3) (layers "F.Cu" "B.Cu") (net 12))
 (via (at 106 98.5) (size 0.6) (drill 0.3) (layers "F.Cu" "B.Cu") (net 12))
 (segment (start 128.5 98.825) (end 128.5 95.5) (width 0.2) (layer "F.Cu") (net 2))
 (segment (start 117.5 104.5) (end 127.5 104.5) (width 0.2) (layer "F.Cu") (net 2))
 (segment (start 127.5 104.5) (end 129.675 102.325) (width 0.2) (layer "F.Cu") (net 2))
 (segment (start 129.675 100) (end 128.5 98.825) (width 0.2) (layer "F.Cu") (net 2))
 (segment (start 129.675 102.325) (end 129.675 100) (width 0.2) (layer "F.Cu") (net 2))
 (segment (start 128.6875 95.5125) (end 129.2 95) (width 0.2) (layer "F.Cu") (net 2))
 (via (at 117.5 104.5) (size 0.6) (drill 0.3) (layers "F.Cu" "B.Cu") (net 2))
 (via (at 120 82.5) (size 0.6) (drill 0.3) (layers "F.Cu" "B.Cu") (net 2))
 (segment (start 136 94.5) (end 136 82.5) (width 0.2) (layer "F.Cu") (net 1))
 (segment (start 134 95) (end 135.5 95) (width 0.2) (layer "F.Cu") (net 1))
 (segment (start 135.5 95) (end 136 94.5) (width 0.2) (layer "F.Cu") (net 1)))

